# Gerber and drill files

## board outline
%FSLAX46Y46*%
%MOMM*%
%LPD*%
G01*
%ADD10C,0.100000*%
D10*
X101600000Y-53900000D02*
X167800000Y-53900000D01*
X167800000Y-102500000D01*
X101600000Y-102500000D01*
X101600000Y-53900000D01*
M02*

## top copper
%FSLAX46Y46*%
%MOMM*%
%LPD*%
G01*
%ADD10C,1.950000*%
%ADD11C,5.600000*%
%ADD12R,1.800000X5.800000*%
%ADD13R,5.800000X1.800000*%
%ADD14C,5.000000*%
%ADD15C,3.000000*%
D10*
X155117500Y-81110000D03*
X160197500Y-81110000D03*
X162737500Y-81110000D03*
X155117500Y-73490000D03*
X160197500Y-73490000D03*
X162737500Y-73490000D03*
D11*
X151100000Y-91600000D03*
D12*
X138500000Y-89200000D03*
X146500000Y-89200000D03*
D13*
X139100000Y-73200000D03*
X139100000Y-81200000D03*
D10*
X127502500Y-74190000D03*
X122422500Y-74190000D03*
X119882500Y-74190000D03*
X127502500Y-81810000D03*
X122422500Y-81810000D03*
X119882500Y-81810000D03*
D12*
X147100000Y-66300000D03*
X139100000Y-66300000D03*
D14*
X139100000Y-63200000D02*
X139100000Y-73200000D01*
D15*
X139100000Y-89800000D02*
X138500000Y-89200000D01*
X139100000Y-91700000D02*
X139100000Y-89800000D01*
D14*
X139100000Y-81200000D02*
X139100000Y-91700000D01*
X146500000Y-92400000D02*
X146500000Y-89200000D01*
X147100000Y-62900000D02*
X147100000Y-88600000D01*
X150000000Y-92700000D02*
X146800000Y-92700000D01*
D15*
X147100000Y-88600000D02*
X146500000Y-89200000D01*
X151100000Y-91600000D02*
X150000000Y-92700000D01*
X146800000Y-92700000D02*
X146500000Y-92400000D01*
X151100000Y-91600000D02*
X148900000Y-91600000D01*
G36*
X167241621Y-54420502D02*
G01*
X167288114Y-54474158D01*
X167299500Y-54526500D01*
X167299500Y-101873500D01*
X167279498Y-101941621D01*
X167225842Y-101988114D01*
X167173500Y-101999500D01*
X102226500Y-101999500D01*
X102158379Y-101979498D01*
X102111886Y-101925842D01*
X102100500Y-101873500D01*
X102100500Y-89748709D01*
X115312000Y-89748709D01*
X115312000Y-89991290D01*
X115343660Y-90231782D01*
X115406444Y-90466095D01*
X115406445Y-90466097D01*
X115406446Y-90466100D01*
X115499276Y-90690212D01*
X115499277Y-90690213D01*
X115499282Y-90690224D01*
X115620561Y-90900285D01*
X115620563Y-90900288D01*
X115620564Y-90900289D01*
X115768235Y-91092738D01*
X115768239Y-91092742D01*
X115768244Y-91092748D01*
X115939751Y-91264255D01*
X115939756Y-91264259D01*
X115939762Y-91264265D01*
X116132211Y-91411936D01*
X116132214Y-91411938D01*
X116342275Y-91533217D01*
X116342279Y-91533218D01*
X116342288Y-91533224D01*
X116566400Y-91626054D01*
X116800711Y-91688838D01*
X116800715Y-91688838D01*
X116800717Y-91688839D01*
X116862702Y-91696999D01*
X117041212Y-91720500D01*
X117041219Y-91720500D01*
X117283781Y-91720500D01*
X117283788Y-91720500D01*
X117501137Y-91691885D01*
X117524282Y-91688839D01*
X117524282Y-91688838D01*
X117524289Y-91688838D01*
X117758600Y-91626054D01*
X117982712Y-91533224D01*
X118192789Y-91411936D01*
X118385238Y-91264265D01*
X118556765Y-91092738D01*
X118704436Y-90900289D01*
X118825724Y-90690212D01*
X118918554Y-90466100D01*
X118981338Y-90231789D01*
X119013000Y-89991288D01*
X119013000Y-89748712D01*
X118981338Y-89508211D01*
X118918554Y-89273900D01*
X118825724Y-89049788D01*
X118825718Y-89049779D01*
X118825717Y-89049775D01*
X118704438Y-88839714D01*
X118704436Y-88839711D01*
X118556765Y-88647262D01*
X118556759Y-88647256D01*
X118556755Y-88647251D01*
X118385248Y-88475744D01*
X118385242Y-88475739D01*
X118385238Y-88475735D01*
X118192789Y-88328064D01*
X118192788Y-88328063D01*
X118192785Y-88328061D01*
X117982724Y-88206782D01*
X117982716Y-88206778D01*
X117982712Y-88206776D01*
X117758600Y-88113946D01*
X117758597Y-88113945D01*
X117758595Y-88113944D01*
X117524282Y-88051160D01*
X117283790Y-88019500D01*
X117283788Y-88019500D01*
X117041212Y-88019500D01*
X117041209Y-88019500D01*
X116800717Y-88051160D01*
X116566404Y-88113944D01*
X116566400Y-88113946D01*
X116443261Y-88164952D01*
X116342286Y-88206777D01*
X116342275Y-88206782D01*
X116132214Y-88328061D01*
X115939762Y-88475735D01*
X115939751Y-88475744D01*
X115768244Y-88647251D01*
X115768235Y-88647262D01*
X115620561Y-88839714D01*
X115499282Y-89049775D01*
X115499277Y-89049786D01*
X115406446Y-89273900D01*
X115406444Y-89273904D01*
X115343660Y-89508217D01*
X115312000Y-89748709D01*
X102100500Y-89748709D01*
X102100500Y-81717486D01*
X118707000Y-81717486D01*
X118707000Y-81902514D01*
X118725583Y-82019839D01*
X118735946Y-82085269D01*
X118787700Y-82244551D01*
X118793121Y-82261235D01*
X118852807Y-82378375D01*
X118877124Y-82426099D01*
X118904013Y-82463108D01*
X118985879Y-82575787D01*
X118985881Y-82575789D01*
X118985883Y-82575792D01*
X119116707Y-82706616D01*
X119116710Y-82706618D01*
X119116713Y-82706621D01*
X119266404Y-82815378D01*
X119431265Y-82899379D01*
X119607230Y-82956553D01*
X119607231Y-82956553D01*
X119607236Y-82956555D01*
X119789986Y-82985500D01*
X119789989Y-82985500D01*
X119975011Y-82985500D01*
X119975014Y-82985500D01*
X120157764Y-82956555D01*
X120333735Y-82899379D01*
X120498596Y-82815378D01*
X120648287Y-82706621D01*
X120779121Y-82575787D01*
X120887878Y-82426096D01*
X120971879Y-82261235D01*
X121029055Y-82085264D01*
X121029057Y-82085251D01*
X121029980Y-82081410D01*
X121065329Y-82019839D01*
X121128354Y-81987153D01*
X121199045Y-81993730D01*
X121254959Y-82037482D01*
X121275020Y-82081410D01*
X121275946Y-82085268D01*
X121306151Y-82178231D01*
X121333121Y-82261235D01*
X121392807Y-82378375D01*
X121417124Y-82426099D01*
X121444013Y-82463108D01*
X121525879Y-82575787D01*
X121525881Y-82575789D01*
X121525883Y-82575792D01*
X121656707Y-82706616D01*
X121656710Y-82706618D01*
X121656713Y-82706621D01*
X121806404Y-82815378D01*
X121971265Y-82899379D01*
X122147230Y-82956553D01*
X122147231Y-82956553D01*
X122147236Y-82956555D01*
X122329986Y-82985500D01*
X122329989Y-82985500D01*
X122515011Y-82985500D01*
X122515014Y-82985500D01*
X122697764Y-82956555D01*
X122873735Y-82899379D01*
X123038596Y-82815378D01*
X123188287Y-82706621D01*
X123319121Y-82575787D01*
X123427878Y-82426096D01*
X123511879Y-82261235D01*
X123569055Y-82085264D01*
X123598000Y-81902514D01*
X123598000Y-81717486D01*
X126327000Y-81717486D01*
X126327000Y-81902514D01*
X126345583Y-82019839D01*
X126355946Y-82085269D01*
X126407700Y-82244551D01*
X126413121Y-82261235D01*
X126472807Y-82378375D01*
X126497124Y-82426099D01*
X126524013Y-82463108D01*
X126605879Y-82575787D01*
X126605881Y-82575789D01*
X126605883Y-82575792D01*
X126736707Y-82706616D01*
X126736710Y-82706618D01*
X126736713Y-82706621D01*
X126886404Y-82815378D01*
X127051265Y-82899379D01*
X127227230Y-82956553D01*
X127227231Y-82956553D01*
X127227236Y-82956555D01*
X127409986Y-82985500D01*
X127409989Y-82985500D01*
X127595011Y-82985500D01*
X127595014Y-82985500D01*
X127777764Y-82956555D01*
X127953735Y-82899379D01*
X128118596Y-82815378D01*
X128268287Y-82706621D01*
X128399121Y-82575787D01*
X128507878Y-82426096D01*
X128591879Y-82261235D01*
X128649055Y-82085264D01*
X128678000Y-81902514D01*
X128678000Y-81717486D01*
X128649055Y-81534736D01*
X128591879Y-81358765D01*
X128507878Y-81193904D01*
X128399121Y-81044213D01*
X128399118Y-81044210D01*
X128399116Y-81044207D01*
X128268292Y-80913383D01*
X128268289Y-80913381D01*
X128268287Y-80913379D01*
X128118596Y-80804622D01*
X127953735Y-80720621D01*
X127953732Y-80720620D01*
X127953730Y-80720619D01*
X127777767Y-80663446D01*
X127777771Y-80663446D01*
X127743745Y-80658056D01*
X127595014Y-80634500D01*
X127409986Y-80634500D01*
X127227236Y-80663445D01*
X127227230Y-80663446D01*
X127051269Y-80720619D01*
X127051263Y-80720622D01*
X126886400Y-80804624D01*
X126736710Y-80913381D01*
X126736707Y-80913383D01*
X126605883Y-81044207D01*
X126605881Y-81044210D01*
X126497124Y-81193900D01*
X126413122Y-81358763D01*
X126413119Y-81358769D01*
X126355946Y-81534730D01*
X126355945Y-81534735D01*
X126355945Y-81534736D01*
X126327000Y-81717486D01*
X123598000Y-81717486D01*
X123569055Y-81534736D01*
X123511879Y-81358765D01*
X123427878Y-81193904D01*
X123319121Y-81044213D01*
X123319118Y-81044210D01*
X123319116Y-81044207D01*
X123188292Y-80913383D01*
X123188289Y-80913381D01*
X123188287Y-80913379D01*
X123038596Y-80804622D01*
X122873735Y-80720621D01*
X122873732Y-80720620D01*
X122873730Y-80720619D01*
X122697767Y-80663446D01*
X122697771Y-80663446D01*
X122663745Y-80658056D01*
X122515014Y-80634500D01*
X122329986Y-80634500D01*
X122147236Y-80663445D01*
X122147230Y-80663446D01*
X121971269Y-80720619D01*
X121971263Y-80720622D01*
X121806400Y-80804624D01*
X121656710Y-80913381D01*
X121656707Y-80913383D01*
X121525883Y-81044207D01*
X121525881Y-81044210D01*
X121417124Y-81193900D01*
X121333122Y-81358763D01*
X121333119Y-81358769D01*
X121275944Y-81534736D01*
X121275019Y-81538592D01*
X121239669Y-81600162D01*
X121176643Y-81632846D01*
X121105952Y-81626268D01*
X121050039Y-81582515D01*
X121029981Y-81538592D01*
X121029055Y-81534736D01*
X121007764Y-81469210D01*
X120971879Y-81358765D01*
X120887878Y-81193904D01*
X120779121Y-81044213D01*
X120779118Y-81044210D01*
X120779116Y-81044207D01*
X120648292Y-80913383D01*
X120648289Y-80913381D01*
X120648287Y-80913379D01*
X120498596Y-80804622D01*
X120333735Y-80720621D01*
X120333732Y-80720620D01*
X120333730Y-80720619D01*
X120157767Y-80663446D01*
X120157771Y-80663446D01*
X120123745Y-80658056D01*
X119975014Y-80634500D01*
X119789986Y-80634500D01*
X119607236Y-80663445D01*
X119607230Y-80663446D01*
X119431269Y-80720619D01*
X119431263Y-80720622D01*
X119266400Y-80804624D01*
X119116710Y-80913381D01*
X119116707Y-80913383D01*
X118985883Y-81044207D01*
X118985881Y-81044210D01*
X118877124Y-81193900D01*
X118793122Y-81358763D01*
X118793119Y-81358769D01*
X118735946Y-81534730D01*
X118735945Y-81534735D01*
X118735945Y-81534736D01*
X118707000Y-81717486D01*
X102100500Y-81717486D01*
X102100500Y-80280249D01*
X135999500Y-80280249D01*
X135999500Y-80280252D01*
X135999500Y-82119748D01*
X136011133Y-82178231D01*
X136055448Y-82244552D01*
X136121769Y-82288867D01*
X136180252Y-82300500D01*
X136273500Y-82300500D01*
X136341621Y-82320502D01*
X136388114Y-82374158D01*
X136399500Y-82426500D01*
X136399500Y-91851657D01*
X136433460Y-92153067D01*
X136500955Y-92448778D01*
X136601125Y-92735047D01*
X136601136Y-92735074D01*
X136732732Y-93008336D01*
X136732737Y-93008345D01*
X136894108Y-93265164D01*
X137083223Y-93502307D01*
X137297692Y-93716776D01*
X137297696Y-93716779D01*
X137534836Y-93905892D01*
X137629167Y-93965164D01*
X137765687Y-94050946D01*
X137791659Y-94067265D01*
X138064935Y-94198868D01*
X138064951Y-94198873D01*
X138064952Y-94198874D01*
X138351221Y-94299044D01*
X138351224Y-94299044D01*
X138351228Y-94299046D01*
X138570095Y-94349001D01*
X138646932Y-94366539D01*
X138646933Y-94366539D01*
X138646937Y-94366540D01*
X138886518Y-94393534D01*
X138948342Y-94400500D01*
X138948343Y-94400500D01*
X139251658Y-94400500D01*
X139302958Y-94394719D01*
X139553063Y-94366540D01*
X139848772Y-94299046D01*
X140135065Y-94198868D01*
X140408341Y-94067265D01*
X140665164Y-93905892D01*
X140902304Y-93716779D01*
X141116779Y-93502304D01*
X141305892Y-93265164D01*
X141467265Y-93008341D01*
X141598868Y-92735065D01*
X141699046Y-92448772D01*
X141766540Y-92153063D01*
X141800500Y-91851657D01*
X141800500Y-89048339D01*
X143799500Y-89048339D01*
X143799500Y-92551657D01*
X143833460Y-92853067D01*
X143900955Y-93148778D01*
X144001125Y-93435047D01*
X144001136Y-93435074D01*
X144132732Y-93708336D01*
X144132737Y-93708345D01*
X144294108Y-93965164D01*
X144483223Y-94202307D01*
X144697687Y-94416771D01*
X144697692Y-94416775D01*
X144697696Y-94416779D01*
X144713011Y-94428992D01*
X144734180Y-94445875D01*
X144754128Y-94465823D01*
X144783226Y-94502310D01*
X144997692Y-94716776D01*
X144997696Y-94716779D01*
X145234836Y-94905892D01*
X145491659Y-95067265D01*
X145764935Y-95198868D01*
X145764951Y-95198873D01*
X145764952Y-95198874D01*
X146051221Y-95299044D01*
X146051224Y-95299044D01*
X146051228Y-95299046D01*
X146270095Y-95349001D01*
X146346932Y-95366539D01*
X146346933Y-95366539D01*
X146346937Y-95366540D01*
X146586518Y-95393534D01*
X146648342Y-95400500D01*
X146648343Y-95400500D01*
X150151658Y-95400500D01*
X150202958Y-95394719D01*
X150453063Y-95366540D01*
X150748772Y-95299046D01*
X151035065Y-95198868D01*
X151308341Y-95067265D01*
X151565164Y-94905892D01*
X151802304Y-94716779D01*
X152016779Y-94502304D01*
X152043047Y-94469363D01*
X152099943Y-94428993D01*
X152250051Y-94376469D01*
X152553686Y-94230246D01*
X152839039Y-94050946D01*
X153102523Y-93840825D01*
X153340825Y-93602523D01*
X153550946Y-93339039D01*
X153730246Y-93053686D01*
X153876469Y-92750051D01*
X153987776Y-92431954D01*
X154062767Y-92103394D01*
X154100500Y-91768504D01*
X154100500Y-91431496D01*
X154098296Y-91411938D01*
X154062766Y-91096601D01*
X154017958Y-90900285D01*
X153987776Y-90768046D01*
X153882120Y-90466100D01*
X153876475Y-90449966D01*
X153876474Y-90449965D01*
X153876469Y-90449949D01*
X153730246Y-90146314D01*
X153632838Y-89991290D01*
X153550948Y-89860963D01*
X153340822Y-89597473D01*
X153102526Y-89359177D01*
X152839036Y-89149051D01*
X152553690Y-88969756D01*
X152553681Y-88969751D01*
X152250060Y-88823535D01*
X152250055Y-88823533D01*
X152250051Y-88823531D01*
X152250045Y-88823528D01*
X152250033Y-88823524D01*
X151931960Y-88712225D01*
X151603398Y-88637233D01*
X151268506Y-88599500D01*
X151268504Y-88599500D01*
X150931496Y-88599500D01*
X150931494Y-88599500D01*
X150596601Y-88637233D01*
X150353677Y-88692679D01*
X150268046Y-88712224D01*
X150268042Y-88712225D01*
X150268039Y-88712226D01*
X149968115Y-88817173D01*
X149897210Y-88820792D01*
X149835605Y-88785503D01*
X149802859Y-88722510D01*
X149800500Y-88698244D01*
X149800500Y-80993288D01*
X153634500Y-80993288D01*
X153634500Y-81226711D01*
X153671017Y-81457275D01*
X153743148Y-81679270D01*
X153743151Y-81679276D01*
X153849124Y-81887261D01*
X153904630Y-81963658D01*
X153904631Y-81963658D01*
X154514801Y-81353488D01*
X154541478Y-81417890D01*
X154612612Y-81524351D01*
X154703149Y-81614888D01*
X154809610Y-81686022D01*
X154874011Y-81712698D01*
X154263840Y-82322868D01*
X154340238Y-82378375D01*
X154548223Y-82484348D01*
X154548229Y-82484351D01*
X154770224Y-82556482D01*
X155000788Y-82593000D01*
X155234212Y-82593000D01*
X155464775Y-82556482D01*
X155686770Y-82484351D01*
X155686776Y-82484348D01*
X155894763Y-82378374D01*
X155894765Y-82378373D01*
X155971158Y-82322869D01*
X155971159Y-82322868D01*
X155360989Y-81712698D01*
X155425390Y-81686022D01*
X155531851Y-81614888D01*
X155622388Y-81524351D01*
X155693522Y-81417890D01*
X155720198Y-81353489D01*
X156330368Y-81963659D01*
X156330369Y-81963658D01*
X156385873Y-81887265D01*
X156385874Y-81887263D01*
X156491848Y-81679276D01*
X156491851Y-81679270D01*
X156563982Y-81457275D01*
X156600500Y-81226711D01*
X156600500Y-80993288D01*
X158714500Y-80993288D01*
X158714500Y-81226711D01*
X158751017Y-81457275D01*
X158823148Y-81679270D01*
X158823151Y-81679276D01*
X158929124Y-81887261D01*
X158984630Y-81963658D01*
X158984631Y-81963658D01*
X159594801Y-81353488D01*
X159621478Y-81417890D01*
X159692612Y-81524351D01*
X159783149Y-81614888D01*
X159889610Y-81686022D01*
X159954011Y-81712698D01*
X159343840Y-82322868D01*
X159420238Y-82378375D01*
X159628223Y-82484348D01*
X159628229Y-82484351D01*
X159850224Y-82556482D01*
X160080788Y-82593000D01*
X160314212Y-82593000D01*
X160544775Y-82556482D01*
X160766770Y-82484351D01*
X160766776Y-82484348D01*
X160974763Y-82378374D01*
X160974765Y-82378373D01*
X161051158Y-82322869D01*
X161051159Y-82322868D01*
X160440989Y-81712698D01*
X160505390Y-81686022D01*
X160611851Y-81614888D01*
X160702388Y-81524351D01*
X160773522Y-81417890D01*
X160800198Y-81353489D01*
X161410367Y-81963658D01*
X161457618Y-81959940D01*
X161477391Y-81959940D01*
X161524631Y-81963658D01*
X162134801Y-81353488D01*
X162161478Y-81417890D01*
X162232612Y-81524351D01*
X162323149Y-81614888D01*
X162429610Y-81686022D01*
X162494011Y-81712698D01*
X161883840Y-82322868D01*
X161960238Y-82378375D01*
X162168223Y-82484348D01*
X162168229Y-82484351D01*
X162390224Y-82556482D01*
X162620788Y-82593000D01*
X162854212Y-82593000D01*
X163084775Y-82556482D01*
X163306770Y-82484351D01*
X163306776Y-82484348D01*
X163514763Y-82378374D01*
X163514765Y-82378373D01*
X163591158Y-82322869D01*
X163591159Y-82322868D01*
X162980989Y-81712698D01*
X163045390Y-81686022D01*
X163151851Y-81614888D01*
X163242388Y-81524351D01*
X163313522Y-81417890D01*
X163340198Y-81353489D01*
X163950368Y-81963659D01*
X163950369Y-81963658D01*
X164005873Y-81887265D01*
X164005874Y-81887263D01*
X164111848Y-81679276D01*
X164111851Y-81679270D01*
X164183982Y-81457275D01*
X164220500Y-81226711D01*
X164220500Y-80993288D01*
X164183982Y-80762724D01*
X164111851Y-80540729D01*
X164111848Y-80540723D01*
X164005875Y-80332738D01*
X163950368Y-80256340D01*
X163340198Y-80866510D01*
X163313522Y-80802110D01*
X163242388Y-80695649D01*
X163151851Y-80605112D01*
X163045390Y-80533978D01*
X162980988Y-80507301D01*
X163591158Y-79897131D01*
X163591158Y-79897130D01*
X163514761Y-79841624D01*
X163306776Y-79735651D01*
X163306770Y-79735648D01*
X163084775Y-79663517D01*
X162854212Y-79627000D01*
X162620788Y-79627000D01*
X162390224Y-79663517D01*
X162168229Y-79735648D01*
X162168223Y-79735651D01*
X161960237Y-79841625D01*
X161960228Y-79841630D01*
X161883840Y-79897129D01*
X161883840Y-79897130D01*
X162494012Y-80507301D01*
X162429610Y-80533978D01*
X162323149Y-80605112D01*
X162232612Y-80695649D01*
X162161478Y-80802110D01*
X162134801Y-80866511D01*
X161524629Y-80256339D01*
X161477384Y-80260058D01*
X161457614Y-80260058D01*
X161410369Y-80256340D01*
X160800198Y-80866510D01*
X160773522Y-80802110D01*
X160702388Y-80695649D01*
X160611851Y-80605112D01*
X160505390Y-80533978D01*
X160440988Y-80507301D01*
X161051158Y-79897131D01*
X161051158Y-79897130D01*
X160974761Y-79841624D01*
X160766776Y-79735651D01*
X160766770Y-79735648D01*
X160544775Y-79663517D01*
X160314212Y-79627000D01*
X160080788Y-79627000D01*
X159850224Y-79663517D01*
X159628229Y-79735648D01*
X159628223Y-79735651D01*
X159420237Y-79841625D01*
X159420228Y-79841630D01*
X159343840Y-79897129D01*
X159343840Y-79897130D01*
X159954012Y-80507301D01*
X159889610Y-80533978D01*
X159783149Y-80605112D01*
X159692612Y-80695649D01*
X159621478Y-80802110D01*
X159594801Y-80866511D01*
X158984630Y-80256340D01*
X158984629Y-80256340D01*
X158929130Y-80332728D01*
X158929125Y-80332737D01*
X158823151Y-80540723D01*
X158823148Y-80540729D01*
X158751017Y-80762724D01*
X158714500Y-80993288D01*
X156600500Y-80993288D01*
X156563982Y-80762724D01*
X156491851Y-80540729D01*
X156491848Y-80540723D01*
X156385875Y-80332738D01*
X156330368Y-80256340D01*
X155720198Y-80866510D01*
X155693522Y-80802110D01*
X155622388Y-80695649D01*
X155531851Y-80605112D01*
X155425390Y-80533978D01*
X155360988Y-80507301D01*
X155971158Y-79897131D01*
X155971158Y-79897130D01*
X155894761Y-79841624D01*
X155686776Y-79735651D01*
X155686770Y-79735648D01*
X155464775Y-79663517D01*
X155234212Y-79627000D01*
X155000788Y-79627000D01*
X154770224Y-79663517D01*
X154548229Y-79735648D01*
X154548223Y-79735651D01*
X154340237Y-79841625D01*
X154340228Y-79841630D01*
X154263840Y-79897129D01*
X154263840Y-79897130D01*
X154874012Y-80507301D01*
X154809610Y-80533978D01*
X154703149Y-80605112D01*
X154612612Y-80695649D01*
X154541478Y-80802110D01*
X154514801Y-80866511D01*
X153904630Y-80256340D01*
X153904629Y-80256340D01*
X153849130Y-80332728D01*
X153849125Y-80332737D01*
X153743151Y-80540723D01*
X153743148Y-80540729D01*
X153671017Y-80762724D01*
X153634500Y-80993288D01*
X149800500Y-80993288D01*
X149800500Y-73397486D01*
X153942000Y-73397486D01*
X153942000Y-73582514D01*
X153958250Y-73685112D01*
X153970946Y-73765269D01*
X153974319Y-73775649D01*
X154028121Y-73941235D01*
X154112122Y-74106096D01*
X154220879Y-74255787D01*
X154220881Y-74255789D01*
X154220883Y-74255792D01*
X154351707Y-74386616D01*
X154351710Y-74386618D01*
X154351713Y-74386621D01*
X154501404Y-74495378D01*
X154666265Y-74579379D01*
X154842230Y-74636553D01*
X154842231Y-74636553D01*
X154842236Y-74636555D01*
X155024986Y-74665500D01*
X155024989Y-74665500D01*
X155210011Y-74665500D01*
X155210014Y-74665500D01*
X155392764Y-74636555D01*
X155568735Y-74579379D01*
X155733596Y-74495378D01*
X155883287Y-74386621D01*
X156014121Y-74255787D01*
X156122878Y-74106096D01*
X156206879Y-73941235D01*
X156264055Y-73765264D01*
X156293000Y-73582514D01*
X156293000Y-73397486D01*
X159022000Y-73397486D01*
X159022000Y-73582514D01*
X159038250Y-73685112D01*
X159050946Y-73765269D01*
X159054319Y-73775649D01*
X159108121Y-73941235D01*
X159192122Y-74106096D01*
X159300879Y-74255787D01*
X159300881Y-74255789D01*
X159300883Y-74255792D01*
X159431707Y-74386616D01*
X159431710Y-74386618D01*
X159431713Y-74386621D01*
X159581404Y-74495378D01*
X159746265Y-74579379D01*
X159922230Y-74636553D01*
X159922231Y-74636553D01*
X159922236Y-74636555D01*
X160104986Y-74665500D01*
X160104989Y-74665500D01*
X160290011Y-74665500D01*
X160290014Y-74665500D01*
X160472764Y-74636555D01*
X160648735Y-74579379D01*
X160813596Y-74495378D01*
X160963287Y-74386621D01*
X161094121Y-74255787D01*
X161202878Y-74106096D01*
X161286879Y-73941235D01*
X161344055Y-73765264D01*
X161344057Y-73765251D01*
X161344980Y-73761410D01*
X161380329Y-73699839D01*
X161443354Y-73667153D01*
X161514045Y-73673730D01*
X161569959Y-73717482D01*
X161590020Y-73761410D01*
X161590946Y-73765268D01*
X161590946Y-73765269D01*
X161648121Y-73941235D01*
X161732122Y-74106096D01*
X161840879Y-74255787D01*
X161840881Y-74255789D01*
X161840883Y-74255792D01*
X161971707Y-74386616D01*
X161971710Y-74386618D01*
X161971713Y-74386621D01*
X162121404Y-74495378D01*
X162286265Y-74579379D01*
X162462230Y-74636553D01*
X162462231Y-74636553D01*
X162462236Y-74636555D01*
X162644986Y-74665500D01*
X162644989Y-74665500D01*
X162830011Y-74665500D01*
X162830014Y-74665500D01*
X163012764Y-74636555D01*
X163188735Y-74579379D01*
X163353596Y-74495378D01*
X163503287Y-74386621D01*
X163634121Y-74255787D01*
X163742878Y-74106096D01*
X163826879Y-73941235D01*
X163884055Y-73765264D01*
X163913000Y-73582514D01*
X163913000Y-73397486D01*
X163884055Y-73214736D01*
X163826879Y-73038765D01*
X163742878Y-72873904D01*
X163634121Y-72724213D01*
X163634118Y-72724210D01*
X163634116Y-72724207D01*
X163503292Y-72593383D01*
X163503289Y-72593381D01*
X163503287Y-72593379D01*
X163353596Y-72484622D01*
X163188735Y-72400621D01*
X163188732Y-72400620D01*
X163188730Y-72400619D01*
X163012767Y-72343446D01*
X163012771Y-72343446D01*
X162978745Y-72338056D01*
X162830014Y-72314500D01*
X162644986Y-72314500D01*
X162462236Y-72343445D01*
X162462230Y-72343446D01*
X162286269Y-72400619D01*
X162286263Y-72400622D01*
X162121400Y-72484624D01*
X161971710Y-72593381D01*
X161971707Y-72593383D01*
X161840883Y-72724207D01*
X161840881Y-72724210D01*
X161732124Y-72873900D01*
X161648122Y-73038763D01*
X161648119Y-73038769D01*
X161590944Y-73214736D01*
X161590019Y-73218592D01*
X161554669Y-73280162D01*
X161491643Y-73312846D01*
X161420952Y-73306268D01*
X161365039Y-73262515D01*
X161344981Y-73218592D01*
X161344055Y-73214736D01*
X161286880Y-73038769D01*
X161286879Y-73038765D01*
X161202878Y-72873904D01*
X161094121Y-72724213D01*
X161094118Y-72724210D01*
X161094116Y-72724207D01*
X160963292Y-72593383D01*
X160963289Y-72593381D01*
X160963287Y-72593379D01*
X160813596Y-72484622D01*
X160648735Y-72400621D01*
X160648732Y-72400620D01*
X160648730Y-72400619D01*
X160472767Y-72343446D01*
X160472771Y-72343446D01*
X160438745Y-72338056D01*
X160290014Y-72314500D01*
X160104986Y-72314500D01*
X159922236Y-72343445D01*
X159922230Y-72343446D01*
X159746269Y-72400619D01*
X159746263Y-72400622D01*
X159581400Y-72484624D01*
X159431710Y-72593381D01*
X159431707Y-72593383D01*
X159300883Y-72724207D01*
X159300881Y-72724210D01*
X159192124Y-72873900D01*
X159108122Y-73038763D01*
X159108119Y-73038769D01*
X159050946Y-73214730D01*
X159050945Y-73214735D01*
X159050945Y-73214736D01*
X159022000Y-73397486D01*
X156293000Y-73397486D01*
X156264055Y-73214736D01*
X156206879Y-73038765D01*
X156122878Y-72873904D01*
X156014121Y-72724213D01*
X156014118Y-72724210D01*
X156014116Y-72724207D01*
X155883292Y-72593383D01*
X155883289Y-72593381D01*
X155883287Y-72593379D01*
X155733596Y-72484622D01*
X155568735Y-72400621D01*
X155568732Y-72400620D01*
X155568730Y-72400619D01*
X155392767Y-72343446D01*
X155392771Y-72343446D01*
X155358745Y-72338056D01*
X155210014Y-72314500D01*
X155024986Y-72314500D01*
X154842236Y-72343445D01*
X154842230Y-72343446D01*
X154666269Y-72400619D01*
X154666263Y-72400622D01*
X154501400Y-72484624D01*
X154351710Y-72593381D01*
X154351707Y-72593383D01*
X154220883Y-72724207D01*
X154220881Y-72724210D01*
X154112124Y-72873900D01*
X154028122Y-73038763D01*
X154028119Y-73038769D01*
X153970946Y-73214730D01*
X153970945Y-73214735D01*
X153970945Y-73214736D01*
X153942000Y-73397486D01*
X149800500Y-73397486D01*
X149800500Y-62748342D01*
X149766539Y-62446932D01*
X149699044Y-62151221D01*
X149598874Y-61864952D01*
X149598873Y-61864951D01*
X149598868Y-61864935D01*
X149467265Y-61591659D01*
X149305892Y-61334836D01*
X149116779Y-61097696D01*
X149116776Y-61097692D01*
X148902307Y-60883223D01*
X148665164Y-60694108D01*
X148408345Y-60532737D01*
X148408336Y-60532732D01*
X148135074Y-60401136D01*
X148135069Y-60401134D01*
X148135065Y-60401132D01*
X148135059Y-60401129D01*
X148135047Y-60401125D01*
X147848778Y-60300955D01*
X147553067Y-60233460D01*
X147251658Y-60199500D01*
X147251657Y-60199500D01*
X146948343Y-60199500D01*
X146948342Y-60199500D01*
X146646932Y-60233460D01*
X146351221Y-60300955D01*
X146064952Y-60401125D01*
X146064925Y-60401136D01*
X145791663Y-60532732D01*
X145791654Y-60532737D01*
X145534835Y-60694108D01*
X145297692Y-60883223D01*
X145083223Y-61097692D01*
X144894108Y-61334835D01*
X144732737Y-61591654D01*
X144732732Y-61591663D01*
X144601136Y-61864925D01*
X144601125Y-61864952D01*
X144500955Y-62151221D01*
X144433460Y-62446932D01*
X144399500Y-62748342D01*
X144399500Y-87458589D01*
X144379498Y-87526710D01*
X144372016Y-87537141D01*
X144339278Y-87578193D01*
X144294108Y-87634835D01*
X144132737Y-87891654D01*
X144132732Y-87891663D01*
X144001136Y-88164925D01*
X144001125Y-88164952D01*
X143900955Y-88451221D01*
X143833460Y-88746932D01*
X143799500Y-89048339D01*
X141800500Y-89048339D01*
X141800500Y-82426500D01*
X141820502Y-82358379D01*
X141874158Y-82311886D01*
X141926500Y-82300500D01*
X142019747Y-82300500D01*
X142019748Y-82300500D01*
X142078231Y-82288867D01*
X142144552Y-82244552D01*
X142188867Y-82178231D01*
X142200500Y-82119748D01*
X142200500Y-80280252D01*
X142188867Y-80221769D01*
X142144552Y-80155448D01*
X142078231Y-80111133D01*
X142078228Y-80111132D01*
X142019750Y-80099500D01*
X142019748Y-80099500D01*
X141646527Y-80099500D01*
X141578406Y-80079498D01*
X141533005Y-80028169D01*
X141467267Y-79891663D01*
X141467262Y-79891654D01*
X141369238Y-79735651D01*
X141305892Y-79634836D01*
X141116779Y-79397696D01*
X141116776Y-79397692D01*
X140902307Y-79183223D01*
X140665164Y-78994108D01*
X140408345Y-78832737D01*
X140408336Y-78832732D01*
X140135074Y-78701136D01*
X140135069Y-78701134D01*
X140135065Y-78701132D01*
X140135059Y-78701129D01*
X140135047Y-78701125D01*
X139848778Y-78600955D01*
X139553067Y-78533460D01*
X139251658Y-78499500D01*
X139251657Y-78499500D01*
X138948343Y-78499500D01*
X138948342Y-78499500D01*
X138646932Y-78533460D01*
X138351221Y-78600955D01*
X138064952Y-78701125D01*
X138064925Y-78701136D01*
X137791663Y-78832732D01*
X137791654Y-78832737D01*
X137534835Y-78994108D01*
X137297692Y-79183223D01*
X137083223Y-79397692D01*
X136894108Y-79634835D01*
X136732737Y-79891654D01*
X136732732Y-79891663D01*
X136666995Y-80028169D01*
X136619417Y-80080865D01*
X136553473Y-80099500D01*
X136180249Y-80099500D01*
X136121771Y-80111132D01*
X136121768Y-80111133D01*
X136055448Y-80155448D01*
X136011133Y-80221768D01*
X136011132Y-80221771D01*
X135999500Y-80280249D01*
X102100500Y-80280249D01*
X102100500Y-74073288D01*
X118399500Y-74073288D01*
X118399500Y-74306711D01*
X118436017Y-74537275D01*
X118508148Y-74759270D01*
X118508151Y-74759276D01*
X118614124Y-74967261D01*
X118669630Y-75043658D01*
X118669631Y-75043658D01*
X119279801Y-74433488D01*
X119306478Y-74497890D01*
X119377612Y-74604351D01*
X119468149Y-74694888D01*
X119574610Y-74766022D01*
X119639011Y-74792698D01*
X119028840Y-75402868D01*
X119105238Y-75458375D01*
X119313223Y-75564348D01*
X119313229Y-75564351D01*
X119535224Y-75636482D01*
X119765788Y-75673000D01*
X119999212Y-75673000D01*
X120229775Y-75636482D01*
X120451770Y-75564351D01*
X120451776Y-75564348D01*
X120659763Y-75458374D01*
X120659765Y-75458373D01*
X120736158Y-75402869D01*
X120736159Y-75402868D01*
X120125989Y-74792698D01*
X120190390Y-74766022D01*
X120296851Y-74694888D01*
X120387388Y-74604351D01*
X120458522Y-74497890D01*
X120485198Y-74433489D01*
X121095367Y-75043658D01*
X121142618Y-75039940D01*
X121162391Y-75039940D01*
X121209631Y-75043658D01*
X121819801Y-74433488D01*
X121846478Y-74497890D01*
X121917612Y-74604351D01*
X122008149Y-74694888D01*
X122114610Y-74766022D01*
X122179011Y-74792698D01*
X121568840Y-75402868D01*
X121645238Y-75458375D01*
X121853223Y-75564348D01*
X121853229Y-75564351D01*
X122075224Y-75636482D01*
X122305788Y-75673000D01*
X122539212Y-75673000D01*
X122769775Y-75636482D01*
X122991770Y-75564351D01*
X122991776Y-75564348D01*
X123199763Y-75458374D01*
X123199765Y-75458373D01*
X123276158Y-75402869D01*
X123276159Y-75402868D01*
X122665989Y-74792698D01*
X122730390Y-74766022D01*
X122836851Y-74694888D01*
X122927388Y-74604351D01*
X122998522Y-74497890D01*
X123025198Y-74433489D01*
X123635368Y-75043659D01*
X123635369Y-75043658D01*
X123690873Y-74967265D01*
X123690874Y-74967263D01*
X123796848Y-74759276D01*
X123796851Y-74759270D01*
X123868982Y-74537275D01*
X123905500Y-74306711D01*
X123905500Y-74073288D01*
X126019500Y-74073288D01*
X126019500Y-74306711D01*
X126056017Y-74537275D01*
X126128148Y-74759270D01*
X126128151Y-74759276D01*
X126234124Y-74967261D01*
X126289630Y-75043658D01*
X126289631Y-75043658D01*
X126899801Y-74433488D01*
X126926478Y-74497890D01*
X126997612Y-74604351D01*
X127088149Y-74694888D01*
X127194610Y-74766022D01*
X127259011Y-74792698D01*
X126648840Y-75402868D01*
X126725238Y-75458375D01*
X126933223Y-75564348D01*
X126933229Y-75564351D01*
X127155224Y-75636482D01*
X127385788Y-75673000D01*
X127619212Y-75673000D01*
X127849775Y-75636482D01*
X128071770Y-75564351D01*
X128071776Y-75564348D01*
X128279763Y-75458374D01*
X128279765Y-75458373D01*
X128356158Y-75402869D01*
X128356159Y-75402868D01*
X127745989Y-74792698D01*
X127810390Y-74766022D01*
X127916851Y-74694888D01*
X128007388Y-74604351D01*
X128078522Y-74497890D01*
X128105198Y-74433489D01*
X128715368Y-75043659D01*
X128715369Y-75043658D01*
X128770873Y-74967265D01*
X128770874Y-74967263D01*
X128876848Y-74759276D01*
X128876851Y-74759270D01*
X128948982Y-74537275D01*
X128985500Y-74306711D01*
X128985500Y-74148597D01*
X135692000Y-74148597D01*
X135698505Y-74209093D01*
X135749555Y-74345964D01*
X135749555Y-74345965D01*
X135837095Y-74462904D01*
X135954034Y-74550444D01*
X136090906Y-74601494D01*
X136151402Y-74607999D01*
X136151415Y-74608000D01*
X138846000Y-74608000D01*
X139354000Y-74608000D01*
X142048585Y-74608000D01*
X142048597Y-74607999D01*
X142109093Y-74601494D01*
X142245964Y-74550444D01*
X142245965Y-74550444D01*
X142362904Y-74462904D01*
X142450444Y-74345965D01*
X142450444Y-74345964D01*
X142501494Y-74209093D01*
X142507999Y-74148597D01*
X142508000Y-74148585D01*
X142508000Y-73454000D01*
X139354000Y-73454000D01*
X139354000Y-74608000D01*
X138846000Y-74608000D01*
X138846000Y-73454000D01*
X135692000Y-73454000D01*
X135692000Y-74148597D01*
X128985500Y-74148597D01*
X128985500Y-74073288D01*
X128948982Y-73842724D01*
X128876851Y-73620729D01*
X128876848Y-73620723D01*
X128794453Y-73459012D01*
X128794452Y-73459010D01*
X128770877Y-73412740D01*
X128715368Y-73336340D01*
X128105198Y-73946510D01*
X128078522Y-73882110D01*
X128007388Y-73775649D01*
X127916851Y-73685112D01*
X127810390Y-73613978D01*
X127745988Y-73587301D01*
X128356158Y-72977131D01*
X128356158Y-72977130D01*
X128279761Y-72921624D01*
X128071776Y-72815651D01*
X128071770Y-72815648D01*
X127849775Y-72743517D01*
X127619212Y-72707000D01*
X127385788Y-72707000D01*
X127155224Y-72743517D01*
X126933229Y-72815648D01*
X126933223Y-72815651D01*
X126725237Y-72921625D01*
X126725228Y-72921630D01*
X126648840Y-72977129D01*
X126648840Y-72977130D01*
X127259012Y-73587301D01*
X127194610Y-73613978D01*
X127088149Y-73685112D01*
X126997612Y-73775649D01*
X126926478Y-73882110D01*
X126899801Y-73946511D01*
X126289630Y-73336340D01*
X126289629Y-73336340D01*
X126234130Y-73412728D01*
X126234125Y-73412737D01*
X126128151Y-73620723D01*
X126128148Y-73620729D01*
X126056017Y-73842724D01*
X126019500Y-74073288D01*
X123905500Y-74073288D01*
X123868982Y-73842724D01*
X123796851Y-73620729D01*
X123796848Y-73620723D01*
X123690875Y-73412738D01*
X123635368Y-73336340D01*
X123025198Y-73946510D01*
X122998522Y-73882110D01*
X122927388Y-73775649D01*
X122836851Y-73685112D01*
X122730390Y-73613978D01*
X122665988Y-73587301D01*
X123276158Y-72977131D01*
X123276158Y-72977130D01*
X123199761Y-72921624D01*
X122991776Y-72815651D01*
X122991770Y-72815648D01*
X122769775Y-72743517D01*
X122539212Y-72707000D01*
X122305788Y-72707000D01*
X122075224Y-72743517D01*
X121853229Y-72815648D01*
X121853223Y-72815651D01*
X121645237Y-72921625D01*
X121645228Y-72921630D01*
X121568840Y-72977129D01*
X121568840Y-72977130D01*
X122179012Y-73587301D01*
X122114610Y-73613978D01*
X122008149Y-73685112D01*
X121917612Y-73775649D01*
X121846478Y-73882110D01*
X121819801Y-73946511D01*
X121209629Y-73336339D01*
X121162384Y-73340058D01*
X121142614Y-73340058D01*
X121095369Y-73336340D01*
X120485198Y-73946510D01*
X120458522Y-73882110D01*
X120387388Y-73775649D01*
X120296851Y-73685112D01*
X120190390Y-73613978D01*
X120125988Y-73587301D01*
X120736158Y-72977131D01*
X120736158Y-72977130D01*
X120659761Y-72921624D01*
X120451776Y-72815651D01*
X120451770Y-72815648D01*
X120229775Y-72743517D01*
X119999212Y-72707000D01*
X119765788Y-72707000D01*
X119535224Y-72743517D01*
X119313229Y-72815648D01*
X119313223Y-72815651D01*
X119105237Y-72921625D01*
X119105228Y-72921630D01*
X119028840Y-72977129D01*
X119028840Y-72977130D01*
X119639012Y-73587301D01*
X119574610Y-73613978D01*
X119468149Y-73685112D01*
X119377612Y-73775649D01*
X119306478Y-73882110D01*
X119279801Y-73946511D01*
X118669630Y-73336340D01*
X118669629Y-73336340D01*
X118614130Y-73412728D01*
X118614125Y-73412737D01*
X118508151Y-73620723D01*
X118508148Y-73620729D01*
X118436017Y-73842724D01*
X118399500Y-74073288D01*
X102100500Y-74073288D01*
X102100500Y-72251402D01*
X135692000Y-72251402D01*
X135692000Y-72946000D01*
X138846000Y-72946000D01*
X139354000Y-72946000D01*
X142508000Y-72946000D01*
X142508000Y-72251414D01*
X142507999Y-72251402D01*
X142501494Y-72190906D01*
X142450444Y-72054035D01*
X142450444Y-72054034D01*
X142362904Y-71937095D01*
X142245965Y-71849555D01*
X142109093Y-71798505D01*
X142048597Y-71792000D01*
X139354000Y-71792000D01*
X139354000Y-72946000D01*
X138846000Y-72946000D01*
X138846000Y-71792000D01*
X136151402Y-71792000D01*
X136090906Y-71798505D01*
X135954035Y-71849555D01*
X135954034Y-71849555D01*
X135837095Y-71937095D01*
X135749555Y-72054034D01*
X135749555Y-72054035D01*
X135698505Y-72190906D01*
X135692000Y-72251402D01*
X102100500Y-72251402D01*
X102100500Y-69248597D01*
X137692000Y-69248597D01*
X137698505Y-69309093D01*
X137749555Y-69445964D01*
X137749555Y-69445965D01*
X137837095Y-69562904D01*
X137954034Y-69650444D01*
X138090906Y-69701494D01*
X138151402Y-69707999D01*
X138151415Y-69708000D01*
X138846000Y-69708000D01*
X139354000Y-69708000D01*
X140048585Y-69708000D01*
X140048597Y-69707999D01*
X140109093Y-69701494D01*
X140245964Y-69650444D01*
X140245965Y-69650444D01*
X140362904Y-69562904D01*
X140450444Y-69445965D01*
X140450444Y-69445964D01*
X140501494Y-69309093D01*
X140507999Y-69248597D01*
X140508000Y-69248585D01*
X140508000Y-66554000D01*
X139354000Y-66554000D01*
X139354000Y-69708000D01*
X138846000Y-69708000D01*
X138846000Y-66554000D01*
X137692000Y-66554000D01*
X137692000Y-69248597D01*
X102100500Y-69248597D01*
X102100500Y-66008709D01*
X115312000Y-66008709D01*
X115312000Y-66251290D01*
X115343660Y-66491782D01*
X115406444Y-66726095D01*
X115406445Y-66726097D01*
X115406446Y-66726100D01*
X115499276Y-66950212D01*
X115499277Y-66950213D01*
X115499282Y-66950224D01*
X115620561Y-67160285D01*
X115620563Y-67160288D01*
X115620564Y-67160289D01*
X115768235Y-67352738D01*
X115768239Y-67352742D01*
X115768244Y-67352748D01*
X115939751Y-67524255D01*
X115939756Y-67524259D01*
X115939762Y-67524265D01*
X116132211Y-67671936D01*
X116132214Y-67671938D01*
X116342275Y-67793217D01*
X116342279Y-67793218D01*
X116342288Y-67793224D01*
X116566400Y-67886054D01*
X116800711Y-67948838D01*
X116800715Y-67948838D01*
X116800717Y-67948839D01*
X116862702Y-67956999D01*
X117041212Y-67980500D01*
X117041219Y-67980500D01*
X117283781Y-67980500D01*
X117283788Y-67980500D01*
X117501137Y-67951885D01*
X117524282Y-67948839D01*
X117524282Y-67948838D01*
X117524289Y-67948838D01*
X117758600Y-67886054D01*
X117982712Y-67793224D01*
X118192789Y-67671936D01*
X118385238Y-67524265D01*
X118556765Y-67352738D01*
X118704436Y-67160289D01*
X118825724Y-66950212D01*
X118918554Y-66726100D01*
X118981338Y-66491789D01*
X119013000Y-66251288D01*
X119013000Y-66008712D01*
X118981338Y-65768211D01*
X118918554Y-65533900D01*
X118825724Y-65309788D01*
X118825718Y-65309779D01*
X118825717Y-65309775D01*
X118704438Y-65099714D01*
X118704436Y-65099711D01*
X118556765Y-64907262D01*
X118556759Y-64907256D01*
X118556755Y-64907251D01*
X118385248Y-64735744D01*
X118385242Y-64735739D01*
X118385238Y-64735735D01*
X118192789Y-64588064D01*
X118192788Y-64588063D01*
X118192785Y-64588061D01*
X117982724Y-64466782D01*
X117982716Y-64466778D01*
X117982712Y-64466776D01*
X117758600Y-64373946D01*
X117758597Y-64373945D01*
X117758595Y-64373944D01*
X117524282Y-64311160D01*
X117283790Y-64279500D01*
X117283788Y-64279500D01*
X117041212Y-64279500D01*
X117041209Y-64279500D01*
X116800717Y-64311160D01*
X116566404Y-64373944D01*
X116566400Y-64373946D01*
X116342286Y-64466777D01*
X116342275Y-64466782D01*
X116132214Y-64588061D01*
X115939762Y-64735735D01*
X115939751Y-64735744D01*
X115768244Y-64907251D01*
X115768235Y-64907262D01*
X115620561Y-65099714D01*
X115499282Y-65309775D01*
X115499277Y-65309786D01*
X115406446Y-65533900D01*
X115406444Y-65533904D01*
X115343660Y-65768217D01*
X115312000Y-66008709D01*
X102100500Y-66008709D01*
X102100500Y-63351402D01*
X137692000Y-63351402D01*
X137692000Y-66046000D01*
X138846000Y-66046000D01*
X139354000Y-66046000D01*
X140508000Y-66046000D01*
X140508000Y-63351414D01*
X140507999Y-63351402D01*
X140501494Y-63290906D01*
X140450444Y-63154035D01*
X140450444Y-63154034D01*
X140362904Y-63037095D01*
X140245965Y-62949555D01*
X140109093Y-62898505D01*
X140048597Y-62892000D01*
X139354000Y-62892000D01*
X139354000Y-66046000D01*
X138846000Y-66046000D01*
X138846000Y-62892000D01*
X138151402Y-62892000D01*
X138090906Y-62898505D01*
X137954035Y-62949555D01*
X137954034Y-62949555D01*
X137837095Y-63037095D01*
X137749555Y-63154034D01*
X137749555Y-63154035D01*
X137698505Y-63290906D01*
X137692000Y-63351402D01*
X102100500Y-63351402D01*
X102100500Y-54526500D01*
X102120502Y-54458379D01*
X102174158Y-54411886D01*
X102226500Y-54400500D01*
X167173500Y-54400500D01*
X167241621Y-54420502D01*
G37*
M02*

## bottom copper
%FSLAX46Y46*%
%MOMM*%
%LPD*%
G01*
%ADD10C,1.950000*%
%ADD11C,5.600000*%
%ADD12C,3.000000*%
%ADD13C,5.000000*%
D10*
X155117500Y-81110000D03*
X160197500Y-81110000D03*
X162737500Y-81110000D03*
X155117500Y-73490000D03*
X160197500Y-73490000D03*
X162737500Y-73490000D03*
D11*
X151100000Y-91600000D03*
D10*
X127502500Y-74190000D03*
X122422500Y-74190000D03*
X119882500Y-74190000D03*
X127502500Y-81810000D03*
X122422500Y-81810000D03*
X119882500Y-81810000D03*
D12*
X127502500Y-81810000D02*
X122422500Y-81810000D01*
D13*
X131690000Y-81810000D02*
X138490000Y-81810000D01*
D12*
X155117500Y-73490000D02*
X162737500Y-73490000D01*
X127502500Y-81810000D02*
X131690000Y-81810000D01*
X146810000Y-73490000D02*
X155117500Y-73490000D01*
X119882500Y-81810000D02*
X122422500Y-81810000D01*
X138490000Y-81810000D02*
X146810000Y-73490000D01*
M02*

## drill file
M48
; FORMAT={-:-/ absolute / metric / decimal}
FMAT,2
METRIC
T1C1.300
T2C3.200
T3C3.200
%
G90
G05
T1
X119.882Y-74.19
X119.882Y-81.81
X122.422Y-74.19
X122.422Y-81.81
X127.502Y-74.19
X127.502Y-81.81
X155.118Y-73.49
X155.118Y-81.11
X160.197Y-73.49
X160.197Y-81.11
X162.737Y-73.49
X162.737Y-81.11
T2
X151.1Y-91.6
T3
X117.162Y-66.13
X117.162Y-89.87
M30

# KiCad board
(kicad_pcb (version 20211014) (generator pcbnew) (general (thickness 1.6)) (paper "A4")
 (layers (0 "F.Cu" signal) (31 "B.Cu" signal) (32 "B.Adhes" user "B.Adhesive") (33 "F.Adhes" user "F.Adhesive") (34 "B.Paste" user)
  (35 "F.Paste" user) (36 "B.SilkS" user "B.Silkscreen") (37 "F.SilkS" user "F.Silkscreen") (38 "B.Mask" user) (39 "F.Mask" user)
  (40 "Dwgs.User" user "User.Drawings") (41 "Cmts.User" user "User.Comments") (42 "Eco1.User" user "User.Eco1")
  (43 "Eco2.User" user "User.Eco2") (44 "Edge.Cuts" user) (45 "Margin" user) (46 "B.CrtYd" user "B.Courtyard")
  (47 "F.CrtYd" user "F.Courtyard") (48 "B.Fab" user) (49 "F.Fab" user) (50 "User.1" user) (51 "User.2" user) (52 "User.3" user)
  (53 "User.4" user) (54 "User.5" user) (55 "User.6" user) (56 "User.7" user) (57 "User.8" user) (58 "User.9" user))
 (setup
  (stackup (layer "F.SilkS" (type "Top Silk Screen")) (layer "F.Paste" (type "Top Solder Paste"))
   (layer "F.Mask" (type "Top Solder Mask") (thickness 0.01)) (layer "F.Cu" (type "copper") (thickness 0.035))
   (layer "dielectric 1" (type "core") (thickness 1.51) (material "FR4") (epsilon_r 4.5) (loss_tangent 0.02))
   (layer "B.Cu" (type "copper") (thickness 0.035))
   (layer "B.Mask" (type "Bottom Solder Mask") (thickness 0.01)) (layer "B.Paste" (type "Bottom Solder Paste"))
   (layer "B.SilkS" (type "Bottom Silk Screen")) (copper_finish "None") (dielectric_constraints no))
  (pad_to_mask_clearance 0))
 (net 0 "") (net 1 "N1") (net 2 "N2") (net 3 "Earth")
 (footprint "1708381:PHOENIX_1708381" (layer "F.Cu") (at 182.6375 84.92 90)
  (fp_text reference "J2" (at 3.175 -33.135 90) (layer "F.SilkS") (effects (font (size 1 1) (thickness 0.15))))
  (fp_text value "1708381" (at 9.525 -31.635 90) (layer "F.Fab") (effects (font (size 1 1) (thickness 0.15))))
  (pad "1_1" thru_hole circle locked (at 3.81 -27.52 90) (size 1.95 1.95) (drill 1.3) (layers *.Cu *.Mask) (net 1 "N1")
   (solder_mask_margin 0.102))
  (pad "1_2" thru_hole circle locked (at 3.81 -22.44 90) (size 1.95 1.95) (drill 1.3) (layers *.Cu *.Mask) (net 1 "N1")
   (solder_mask_margin 0.102))
  (pad "1_3" thru_hole circle locked (at 3.81 -19.9 90) (size 1.95 1.95) (drill 1.3) (layers *.Cu *.Mask) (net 1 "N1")
   (solder_mask_margin 0.102))
  (pad "2_1" thru_hole circle locked (at 11.43 -27.52 90) (size 1.95 1.95) (drill 1.3) (layers *.Cu *.Mask) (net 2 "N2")
   (solder_mask_margin 0.102))
  (pad "2_2" thru_hole circle locked (at 11.43 -22.44 90) (size 1.95 1.95) (drill 1.3) (layers *.Cu *.Mask) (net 2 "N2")
   (solder_mask_margin 0.102))
  (pad "2_3" thru_hole circle locked (at 11.43 -19.9 90) (size 1.95 1.95) (drill 1.3) (layers *.Cu *.Mask) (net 2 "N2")
   (solder_mask_margin 0.102)))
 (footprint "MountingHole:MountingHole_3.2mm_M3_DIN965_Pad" (layer "F.Cu") (at 151.1 91.6)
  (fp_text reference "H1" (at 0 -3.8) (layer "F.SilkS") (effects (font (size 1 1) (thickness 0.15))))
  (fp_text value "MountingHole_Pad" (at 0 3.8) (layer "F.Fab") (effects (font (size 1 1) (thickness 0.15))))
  (pad "1" thru_hole circle (at 0 0) (size 5.6 5.6) (drill 3.2) (layers *.Cu *.Mask) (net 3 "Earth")))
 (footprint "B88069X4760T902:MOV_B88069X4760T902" (layer "F.Cu") (at 142.5 89.2)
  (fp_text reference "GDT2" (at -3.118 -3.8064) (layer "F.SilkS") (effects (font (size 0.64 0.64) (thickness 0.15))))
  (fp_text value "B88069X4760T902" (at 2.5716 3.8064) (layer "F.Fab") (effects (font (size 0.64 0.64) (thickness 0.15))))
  (pad "1" smd rect locked (at -4 0) (size 1.8 5.8) (layers "F.Cu" "F.Paste" "F.Mask") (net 2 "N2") (solder_mask_margin 0.102))
  (pad "2" smd rect locked (at 4 0) (size 1.8 5.8) (layers "F.Cu" "F.Paste" "F.Mask") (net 3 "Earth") (solder_mask_margin 0.102)))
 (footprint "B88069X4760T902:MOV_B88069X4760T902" (layer "F.Cu") (at 139.1 77.2 -90)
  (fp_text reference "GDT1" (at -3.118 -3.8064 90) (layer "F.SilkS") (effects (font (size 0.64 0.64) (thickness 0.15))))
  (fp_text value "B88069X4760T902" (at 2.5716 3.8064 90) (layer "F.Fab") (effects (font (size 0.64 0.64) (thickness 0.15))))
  (pad "1" smd rect locked (at -4 0 270) (size 1.8 5.8) (layers "F.Cu" "F.Paste" "F.Mask") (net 1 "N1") (solder_mask_margin 0.102))
  (pad "2" smd rect locked (at 4 0 270) (size 1.8 5.8) (layers "F.Cu" "F.Paste" "F.Mask") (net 2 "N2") (solder_mask_margin 0.102)))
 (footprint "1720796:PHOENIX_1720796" (layer "F.Cu") (at 100.1625 62.33 -90)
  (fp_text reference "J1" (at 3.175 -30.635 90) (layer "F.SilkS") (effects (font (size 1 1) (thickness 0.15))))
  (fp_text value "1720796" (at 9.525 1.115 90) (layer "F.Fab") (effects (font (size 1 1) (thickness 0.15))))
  (pad "" np_thru_hole circle locked (at 27.54 -17 270) (size 3.2 3.2) (drill 3.2) (layers *.Cu *.Mask))
  (pad "" np_thru_hole circle locked (at 3.8 -17 270) (size 3.2 3.2) (drill 3.2) (layers *.Cu *.Mask))
  (pad "1_1" thru_hole circle locked (at 11.86 -27.34 270) (size 1.95 1.95) (drill 1.3) (layers *.Cu *.Mask) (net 1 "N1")
   (solder_mask_margin 0.102))
  (pad "1_2" thru_hole circle locked (at 11.86 -22.26 270) (size 1.95 1.95) (drill 1.3) (layers *.Cu *.Mask) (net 1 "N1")
   (solder_mask_margin 0.102))
  (pad "1_3" thru_hole circle locked (at 11.86 -19.72 270) (size 1.95 1.95) (drill 1.3) (layers *.Cu *.Mask) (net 1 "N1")
   (solder_mask_margin 0.102))
  (pad "2_1" thru_hole circle locked (at 19.48 -27.34 270) (size 1.95 1.95) (drill 1.3) (layers *.Cu *.Mask) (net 2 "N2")
   (solder_mask_margin 0.102))
  (pad "2_2" thru_hole circle locked (at 19.48 -22.26 270) (size 1.95 1.95) (drill 1.3) (layers *.Cu *.Mask) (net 2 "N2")
   (solder_mask_margin 0.102))
  (pad "2_3" thru_hole circle locked (at 19.48 -19.72 270) (size 1.95 1.95) (drill 1.3) (layers *.Cu *.Mask) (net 2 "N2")
   (solder_mask_margin 0.102)))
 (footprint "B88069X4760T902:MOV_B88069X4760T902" (layer "F.Cu") (at 143.1 66.3 180)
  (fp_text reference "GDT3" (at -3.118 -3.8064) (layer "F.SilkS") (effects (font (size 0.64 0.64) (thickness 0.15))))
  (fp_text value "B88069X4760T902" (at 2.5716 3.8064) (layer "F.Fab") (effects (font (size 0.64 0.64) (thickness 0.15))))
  (pad "1" smd rect locked (at -4 0 180) (size 1.8 5.8) (layers "F.Cu" "F.Paste" "F.Mask") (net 3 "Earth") (solder_mask_margin 0.102))
  (pad "2" smd rect locked (at 4 0 180) (size 1.8 5.8) (layers "F.Cu" "F.Paste" "F.Mask") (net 1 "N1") (solder_mask_margin 0.102)))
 (gr_rect (start 101.6 53.9) (end 167.8 102.5) (layer "Edge.Cuts") (width 0.1) (fill none))
 (segment (start 139.1 63.2) (end 139.1 73.2) (width 5) (layer "F.Cu") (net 1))
 (segment (start 139.1 89.8) (end 138.5 89.2) (width 3) (layer "F.Cu") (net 2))
 (segment (start 139.1 91.7) (end 139.1 89.8) (width 3) (layer "F.Cu") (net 2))
 (segment (start 139.1 81.2) (end 139.1 91.7) (width 5) (layer "F.Cu") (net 2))
 (segment (start 127.5025 81.81) (end 122.4225 81.81) (width 3) (layer "B.Cu") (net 2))
 (segment (start 131.69 81.81) (end 138.49 81.81) (width 5) (layer "B.Cu") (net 2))
 (segment (start 155.1175 73.49) (end 162.7375 73.49) (width 3) (layer "B.Cu") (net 2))
 (segment (start 127.5025 81.81) (end 131.69 81.81) (width 3) (layer "B.Cu") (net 2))
 (segment (start 146.81 73.49) (end 155.1175 73.49) (width 3) (layer "B.Cu") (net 2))
 (segment (start 119.8825 81.81) (end 122.4225 81.81) (width 3) (layer "B.Cu") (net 2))
 (segment (start 138.49 81.81) (end 146.81 73.49) (width 3) (layer "B.Cu") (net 2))
 (segment (start 146.5 92.4) (end 146.5 89.2) (width 5) (layer "F.Cu") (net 3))
 (segment (start 147.1 62.9) (end 147.1 88.6) (width 5) (layer "F.Cu") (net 3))
 (segment (start 150 92.7) (end 146.8 92.7) (width 5) (layer "F.Cu") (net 3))
 (segment (start 147.1 88.6) (end 146.5 89.2) (width 3) (layer "F.Cu") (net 3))
 (segment (start 151.1 91.6) (end 150 92.7) (width 3) (layer "F.Cu") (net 3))
 (segment (start 146.8 92.7) (end 146.5 92.4) (width 3) (layer "F.Cu") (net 3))
 (segment (start 151.1 91.6) (end 148.9 91.6) (width 3) (layer "F.Cu") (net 3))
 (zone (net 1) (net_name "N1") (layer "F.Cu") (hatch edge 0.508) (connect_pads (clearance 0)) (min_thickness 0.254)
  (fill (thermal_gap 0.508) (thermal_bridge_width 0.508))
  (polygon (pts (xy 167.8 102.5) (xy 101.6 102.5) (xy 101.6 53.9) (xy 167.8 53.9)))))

